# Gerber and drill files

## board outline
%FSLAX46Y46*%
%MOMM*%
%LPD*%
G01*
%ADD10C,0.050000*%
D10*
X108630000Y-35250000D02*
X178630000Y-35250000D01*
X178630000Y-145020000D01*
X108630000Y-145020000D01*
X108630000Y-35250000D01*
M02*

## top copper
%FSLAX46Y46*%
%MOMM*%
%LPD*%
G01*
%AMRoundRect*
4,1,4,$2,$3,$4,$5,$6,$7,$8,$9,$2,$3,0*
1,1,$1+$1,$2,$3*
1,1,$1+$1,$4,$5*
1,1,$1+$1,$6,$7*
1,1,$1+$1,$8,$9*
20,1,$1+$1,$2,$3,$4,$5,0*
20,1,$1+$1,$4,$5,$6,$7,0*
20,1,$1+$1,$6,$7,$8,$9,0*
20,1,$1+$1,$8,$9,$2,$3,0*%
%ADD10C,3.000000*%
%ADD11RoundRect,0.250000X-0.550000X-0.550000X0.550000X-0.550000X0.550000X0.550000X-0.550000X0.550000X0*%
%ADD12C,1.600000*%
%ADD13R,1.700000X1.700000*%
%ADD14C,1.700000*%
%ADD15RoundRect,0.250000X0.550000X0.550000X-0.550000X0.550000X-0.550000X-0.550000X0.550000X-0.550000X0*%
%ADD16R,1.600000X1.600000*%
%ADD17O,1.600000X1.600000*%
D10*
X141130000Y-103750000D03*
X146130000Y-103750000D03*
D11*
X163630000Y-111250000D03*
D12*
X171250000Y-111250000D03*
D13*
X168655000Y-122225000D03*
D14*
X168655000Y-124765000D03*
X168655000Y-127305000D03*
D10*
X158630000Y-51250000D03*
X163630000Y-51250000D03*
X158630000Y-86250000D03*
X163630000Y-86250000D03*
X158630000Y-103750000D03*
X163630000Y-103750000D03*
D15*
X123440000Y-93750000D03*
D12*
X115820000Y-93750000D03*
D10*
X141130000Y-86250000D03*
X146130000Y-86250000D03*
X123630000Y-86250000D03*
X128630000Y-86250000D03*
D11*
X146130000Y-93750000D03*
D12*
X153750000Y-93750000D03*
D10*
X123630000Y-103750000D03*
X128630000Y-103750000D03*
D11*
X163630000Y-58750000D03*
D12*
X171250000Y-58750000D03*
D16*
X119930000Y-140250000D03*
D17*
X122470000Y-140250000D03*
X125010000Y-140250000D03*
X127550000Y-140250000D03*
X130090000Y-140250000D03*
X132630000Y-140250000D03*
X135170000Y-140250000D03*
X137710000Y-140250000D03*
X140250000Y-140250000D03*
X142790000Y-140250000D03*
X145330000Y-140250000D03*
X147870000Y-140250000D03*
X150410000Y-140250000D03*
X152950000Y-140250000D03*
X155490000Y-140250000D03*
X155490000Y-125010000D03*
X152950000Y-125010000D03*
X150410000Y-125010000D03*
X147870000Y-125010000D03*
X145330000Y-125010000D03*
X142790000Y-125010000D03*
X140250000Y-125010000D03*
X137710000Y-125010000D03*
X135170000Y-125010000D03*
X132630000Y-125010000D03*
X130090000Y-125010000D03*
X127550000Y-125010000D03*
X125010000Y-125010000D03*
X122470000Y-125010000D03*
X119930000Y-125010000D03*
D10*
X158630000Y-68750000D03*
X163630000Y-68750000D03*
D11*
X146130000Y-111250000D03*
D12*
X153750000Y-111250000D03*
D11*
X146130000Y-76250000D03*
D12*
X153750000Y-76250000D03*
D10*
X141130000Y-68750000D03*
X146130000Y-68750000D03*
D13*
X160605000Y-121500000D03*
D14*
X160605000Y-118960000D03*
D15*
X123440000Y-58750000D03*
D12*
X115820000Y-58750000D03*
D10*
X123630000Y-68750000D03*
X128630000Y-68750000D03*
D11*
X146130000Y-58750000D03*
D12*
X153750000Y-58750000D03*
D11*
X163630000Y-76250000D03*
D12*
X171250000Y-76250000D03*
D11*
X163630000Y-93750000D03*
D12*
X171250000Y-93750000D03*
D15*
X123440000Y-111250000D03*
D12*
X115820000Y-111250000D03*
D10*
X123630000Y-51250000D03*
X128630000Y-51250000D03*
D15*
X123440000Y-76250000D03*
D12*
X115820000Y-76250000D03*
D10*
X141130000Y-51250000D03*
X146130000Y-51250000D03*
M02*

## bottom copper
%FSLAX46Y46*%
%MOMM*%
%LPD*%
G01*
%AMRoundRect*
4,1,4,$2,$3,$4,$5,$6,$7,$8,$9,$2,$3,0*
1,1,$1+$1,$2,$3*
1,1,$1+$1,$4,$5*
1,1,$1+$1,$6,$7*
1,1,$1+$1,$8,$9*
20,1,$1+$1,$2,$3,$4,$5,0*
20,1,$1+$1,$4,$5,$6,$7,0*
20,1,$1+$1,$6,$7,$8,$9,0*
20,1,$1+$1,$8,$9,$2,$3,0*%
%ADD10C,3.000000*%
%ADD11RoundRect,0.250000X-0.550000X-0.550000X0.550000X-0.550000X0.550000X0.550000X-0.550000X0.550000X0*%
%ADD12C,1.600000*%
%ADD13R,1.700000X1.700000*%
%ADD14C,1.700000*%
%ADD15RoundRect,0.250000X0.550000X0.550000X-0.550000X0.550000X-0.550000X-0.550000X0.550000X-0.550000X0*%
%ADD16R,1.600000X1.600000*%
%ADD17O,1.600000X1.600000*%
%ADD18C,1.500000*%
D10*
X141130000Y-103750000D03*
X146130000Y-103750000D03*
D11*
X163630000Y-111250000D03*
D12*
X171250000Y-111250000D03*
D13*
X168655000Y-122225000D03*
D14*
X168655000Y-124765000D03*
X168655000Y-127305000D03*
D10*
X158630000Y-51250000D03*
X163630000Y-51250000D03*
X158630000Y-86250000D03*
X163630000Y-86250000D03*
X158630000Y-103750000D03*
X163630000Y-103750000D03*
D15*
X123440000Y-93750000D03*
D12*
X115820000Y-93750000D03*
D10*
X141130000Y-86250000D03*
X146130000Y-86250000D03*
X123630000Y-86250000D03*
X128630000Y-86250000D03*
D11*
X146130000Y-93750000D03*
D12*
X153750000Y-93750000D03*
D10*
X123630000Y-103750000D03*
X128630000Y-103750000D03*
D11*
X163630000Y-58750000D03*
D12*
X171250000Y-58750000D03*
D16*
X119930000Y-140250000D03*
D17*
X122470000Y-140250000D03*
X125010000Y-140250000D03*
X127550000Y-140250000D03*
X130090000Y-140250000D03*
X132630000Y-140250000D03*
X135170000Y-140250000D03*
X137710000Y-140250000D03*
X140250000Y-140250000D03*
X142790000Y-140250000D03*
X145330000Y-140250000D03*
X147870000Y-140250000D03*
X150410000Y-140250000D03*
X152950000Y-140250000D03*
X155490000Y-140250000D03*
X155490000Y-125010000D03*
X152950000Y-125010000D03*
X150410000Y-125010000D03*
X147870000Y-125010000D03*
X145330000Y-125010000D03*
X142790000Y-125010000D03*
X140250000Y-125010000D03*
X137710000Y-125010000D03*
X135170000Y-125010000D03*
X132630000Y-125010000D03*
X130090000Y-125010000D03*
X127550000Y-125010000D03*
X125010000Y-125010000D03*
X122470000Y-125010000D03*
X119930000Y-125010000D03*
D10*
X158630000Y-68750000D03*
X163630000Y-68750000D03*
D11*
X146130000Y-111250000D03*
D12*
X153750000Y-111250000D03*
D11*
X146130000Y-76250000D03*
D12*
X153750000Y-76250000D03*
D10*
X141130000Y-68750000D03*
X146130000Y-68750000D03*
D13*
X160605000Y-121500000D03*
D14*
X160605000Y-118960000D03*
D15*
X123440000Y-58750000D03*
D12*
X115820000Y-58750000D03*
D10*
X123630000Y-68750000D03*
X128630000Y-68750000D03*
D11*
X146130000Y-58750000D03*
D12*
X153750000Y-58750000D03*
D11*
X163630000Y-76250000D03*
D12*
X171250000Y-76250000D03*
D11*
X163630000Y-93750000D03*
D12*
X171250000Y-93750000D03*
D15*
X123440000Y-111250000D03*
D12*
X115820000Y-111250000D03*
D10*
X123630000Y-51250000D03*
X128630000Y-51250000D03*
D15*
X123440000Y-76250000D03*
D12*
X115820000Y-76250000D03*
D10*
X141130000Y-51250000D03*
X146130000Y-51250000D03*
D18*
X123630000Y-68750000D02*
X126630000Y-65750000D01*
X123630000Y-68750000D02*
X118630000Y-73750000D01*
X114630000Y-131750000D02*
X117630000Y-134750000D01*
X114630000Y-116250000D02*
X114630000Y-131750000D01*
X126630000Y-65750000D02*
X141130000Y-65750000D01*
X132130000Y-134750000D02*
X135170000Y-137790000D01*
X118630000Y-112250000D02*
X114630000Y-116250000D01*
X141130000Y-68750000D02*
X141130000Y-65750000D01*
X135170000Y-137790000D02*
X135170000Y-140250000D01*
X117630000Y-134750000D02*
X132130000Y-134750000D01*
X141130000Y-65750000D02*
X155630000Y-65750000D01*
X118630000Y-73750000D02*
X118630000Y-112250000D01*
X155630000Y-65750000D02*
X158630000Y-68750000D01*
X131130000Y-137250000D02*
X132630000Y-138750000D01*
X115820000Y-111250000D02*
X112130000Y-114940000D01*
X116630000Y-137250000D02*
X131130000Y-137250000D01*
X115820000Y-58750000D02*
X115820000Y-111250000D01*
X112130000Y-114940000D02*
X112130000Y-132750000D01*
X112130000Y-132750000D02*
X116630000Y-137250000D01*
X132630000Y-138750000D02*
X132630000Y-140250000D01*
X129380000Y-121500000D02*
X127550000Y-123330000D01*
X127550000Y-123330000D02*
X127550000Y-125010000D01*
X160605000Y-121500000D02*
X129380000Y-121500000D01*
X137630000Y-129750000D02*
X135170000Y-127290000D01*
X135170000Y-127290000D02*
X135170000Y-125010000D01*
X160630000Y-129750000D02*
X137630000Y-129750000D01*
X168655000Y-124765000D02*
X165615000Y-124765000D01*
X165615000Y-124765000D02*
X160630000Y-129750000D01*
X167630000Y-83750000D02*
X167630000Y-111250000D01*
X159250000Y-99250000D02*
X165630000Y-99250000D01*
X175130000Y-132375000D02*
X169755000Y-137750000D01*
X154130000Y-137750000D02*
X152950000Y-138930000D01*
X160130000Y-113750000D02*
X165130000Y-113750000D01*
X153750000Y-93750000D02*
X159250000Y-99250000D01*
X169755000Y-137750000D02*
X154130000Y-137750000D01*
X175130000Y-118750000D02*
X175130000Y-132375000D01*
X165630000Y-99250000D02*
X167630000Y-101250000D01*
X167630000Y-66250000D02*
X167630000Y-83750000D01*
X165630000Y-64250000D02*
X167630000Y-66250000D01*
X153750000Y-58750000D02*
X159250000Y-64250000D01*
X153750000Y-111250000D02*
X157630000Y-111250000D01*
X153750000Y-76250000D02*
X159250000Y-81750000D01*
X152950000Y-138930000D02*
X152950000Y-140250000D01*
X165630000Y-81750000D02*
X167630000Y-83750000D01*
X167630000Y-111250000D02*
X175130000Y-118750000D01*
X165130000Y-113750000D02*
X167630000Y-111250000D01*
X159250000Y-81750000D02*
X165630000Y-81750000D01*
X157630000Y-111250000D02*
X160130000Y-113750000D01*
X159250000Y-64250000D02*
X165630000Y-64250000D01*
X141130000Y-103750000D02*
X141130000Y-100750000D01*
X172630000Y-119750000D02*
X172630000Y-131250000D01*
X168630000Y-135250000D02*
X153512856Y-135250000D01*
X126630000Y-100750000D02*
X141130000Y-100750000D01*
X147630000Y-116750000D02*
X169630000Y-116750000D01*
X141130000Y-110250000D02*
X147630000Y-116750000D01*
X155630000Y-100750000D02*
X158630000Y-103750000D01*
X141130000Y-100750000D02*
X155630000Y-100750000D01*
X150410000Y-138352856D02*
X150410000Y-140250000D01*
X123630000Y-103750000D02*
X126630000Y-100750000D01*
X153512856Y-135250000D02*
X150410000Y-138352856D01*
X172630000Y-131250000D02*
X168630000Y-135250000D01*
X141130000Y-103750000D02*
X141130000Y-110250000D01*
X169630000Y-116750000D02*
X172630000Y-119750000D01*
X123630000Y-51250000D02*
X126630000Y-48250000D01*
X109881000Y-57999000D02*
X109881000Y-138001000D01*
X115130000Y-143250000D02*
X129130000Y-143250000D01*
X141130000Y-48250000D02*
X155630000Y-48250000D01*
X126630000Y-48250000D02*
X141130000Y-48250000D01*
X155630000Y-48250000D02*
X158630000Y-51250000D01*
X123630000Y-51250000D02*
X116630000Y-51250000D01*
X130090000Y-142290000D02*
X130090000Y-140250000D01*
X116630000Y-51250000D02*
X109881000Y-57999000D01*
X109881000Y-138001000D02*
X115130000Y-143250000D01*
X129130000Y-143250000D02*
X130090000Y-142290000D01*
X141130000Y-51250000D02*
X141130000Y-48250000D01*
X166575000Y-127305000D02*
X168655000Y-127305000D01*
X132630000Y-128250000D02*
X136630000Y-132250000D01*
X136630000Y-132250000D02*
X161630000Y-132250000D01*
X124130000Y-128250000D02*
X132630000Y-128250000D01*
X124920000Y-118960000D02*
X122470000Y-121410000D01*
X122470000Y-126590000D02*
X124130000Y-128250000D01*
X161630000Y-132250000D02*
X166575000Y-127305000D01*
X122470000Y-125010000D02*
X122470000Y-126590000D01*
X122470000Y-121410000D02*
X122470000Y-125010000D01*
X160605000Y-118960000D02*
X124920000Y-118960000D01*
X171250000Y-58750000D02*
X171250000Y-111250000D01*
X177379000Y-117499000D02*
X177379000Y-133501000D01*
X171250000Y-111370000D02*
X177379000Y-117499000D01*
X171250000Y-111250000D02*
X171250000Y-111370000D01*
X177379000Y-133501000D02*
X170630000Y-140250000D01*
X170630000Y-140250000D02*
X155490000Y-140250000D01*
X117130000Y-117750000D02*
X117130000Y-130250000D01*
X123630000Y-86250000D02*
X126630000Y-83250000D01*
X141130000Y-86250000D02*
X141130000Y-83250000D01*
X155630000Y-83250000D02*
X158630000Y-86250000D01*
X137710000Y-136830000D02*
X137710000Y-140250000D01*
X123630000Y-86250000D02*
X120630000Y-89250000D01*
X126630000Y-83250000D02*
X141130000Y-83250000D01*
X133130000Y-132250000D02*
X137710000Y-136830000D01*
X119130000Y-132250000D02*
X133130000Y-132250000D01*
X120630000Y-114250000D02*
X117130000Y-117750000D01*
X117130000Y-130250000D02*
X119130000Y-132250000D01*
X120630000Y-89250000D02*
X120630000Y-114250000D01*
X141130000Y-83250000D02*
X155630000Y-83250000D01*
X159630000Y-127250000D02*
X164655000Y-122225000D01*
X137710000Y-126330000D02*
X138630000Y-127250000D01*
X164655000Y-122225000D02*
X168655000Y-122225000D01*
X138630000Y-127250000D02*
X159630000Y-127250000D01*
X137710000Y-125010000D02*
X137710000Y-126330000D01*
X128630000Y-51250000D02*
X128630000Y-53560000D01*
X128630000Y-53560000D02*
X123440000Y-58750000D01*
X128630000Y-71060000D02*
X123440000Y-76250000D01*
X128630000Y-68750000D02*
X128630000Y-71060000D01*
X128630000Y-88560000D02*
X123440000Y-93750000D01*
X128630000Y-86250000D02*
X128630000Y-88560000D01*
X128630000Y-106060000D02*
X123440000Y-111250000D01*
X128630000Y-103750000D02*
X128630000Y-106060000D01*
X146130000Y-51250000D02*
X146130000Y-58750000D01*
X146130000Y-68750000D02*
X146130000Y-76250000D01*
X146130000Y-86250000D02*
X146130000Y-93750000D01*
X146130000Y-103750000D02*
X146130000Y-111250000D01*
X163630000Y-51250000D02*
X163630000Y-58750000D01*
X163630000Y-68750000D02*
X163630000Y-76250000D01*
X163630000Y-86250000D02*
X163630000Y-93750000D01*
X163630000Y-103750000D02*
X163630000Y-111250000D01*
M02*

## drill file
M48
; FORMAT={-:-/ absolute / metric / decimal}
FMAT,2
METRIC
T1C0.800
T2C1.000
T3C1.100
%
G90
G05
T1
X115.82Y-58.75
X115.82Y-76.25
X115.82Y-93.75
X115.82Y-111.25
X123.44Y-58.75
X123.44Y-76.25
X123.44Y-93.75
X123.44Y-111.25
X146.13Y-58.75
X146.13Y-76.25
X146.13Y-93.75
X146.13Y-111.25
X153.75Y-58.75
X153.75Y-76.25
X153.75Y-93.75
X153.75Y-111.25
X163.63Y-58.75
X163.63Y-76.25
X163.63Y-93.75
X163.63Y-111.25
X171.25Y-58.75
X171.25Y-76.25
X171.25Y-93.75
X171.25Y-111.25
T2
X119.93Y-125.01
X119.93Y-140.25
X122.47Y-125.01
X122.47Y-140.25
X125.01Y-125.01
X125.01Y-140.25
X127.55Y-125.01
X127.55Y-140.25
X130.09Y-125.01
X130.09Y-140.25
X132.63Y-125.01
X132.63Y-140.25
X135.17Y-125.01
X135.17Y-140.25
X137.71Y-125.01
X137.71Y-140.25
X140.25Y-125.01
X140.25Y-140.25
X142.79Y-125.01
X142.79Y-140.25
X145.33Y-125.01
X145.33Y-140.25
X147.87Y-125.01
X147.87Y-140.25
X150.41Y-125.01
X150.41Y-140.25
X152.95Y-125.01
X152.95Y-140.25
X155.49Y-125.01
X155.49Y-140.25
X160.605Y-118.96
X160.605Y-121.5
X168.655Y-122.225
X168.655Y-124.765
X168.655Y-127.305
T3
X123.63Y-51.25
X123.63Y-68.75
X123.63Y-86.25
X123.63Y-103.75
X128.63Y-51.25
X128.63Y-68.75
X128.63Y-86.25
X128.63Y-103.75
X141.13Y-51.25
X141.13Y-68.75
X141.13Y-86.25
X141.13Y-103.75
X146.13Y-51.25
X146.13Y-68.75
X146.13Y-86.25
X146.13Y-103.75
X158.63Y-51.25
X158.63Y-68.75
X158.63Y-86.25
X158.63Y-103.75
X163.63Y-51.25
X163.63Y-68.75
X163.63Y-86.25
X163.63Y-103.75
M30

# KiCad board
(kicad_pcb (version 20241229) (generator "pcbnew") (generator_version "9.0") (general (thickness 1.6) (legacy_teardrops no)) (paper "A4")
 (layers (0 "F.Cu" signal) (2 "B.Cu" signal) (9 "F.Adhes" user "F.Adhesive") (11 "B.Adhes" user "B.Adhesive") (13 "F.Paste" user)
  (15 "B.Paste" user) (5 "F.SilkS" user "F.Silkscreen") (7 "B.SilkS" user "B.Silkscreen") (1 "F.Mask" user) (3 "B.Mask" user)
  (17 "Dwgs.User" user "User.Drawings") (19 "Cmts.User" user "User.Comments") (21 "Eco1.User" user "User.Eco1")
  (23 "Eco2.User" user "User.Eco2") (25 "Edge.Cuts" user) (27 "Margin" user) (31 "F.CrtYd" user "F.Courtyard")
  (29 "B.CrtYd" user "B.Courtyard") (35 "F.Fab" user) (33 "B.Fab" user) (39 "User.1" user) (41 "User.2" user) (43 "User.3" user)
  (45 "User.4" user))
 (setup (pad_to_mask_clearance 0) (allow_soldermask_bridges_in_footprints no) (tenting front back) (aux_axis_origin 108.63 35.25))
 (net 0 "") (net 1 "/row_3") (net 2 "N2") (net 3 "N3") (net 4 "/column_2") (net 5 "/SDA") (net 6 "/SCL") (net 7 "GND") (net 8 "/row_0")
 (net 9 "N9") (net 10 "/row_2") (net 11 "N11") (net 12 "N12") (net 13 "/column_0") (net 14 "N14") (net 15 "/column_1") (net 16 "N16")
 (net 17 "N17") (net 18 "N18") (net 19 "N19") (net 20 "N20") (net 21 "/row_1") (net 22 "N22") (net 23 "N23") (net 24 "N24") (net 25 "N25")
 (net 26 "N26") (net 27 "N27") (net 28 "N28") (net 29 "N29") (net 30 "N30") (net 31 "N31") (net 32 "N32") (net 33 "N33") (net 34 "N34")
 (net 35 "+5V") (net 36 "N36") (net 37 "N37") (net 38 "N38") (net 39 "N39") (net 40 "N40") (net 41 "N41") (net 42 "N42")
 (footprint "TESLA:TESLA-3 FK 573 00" (layer "F.Cu") (at 143.63 103.75)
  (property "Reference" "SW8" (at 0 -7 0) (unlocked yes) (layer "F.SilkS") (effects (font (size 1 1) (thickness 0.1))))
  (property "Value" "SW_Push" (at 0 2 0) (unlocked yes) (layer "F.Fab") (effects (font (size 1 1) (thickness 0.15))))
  (pad "1" thru_hole circle (at -2.5 0) (size 3 3) (drill 1.1) (layers "*.Cu" "*.Mask") (remove_unused_layers no) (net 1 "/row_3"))
  (pad "2" thru_hole circle (at 2.5 0) (size 3 3) (drill 1.1) (layers "*.Cu" "*.Mask") (remove_unused_layers no) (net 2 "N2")))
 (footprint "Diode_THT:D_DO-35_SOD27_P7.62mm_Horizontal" (layer "F.Cu") (at 163.63 111.25)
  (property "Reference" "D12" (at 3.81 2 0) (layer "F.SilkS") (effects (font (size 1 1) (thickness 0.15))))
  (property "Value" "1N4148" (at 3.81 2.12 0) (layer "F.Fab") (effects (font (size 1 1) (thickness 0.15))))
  (pad "1" thru_hole roundrect (at 0 0) (size 1.6 1.6) (drill 0.8) (layers "*.Cu" "*.Mask") (remove_unused_layers no)
   (roundrect_rratio 0.15625) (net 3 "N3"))
  (pad "2" thru_hole circle (at 7.62 0) (size 1.6 1.6) (drill 0.8) (layers "*.Cu" "*.Mask") (remove_unused_layers no) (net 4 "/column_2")))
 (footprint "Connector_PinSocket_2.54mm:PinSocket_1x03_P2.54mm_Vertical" (layer "F.Cu") (at 168.655 122.225)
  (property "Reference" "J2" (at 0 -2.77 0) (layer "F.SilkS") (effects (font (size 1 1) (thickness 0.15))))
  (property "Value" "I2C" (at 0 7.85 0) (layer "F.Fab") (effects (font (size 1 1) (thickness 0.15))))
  (pad "1" thru_hole rect (at 0 0) (size 1.7 1.7) (drill 1) (layers "*.Cu" "*.Mask") (remove_unused_layers no) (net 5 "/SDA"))
  (pad "2" thru_hole circle (at 0 2.54) (size 1.7 1.7) (drill 1) (layers "*.Cu" "*.Mask") (remove_unused_layers no) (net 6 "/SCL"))
  (pad "3" thru_hole circle (at 0 5.08) (size 1.7 1.7) (drill 1) (layers "*.Cu" "*.Mask") (remove_unused_layers no) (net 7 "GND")))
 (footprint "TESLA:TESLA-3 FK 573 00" (layer "F.Cu") (at 161.13 51.25)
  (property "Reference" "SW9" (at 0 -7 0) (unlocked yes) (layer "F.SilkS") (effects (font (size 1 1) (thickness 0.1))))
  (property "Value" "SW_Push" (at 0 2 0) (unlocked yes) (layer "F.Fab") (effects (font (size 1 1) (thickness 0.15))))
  (pad "1" thru_hole circle (at -2.5 0) (size 3 3) (drill 1.1) (layers "*.Cu" "*.Mask") (remove_unused_layers no) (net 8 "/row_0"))
  (pad "2" thru_hole circle (at 2.5 0) (size 3 3) (drill 1.1) (layers "*.Cu" "*.Mask") (remove_unused_layers no) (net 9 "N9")))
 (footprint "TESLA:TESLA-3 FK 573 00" (layer "F.Cu") (at 161.13 86.25)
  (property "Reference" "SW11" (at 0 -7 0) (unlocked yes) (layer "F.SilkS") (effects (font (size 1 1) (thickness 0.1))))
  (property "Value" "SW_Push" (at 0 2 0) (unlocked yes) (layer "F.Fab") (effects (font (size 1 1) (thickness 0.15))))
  (pad "1" thru_hole circle (at -2.5 0) (size 3 3) (drill 1.1) (layers "*.Cu" "*.Mask") (remove_unused_layers no) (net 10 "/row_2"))
  (pad "2" thru_hole circle (at 2.5 0) (size 3 3) (drill 1.1) (layers "*.Cu" "*.Mask") (remove_unused_layers no) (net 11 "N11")))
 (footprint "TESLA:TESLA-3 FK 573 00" (layer "F.Cu") (at 161.13 103.75)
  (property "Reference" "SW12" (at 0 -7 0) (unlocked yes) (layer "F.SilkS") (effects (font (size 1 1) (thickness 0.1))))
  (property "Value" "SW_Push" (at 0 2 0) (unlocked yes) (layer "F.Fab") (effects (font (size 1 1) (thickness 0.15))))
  (pad "1" thru_hole circle (at -2.5 0) (size 3 3) (drill 1.1) (layers "*.Cu" "*.Mask") (remove_unused_layers no) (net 1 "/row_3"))
  (pad "2" thru_hole circle (at 2.5 0) (size 3 3) (drill 1.1) (layers "*.Cu" "*.Mask") (remove_unused_layers no) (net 3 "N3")))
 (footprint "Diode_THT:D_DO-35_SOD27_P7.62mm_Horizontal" (layer "F.Cu") (at 123.44 93.75 180)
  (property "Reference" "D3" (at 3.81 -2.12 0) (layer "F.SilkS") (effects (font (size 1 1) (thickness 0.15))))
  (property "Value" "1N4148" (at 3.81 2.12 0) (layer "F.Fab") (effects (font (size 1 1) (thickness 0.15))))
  (pad "1" thru_hole roundrect (at 0 0 180) (size 1.6 1.6) (drill 0.8) (layers "*.Cu" "*.Mask") (remove_unused_layers no)
   (roundrect_rratio 0.15625) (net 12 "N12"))
  (pad "2" thru_hole circle (at 7.62 0 180) (size 1.6 1.6) (drill 0.8) (layers "*.Cu" "*.Mask") (remove_unused_layers no)
   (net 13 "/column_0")))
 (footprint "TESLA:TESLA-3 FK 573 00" (layer "F.Cu") (at 143.63 86.25)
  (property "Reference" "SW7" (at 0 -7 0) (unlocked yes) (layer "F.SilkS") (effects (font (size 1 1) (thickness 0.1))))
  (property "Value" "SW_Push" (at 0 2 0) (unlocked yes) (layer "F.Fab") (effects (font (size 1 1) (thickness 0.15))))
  (pad "1" thru_hole circle (at -2.5 0) (size 3 3) (drill 1.1) (layers "*.Cu" "*.Mask") (remove_unused_layers no) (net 10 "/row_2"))
  (pad "2" thru_hole circle (at 2.5 0) (size 3 3) (drill 1.1) (layers "*.Cu" "*.Mask") (remove_unused_layers no) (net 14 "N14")))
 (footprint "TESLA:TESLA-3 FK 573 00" (layer "F.Cu") (at 126.13 86.25)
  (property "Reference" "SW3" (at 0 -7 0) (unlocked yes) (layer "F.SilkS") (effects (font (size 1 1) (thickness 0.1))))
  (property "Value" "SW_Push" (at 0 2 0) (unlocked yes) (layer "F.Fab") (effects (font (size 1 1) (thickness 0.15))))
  (pad "1" thru_hole circle (at -2.5 0) (size 3 3) (drill 1.1) (layers "*.Cu" "*.Mask") (remove_unused_layers no) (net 10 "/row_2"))
  (pad "2" thru_hole circle (at 2.5 0) (size 3 3) (drill 1.1) (layers "*.Cu" "*.Mask") (remove_unused_layers no) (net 12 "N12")))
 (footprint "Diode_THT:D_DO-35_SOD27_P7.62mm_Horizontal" (layer "F.Cu") (at 146.13 93.75)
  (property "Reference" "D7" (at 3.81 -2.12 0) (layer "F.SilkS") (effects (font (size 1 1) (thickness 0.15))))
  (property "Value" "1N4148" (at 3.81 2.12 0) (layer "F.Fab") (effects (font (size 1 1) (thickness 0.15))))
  (pad "1" thru_hole roundrect (at 0 0) (size 1.6 1.6) (drill 0.8) (layers "*.Cu" "*.Mask") (remove_unused_layers no)
   (roundrect_rratio 0.15625) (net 14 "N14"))
  (pad "2" thru_hole circle (at 7.62 0) (size 1.6 1.6) (drill 0.8) (layers "*.Cu" "*.Mask") (remove_unused_layers no) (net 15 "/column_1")))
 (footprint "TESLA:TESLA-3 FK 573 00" (layer "F.Cu") (at 126.13 103.75)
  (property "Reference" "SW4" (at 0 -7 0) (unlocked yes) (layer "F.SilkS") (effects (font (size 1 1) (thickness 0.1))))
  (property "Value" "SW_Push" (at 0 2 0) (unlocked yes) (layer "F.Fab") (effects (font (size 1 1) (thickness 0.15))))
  (pad "1" thru_hole circle (at -2.5 0) (size 3 3) (drill 1.1) (layers "*.Cu" "*.Mask") (remove_unused_layers no) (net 1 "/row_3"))
  (pad "2" thru_hole circle (at 2.5 0) (size 3 3) (drill 1.1) (layers "*.Cu" "*.Mask") (remove_unused_layers no) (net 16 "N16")))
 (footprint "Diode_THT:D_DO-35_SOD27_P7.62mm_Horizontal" (layer "F.Cu") (at 163.63 58.75)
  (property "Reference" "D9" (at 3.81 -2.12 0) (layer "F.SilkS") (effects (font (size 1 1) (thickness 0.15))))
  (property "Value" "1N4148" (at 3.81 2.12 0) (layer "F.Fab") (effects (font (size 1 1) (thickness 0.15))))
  (pad "1" thru_hole roundrect (at 0 0) (size 1.6 1.6) (drill 0.8) (layers "*.Cu" "*.Mask") (remove_unused_layers no)
   (roundrect_rratio 0.15625) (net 9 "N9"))
  (pad "2" thru_hole circle (at 7.62 0) (size 1.6 1.6) (drill 0.8) (layers "*.Cu" "*.Mask") (remove_unused_layers no) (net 4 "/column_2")))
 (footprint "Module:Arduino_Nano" (layer "F.Cu") (at 119.93 140.25 90)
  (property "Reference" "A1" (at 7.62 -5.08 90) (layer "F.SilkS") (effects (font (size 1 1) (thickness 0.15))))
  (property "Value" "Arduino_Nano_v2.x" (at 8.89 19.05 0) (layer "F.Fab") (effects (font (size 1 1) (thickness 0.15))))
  (pad "1" thru_hole rect (at 0 0 90) (size 1.6 1.6) (drill 1) (layers "*.Cu" "*.Mask") (remove_unused_layers no) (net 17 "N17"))
  (pad "2" thru_hole oval (at 0 2.54 90) (size 1.6 1.6) (drill 1) (layers "*.Cu" "*.Mask") (remove_unused_layers no) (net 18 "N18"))
  (pad "3" thru_hole oval (at 0 5.08 90) (size 1.6 1.6) (drill 1) (layers "*.Cu" "*.Mask") (remove_unused_layers no) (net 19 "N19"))
  (pad "4" thru_hole oval (at 0 7.62 90) (size 1.6 1.6) (drill 1) (layers "*.Cu" "*.Mask") (remove_unused_layers no) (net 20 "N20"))
  (pad "5" thru_hole oval (at 0 10.16 90) (size 1.6 1.6) (drill 1) (layers "*.Cu" "*.Mask") (remove_unused_layers no) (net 8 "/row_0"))
  (pad "6" thru_hole oval (at 0 12.7 90) (size 1.6 1.6) (drill 1) (layers "*.Cu" "*.Mask") (remove_unused_layers no) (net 13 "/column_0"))
  (pad "7" thru_hole oval (at 0 15.24 90) (size 1.6 1.6) (drill 1) (layers "*.Cu" "*.Mask") (remove_unused_layers no) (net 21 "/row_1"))
  (pad "8" thru_hole oval (at 0 17.78 90) (size 1.6 1.6) (drill 1) (layers "*.Cu" "*.Mask") (remove_unused_layers no) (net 10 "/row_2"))
  (pad "9" thru_hole oval (at 0 20.32 90) (size 1.6 1.6) (drill 1) (layers "*.Cu" "*.Mask") (remove_unused_layers no) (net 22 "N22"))
  (pad "10" thru_hole oval (at 0 22.86 90) (size 1.6 1.6) (drill 1) (layers "*.Cu" "*.Mask") (remove_unused_layers no) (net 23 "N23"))
  (pad "11" thru_hole oval (at 0 25.4 90) (size 1.6 1.6) (drill 1) (layers "*.Cu" "*.Mask") (remove_unused_layers no) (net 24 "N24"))
  (pad "12" thru_hole oval (at 0 27.94 90) (size 1.6 1.6) (drill 1) (layers "*.Cu" "*.Mask") (remove_unused_layers no) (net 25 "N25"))
  (pad "13" thru_hole oval (at 0 30.48 90) (size 1.6 1.6) (drill 1) (layers "*.Cu" "*.Mask") (remove_unused_layers no) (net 1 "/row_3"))
  (pad "14" thru_hole oval (at 0 33.02 90) (size 1.6 1.6) (drill 1) (layers "*.Cu" "*.Mask") (remove_unused_layers no) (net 15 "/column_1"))
  (pad "15" thru_hole oval (at 0 35.56 90) (size 1.6 1.6) (drill 1) (layers "*.Cu" "*.Mask") (remove_unused_layers no) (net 4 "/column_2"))
  (pad "16" thru_hole oval (at 15.24 35.56 90) (size 1.6 1.6) (drill 1) (layers "*.Cu" "*.Mask") (remove_unused_layers no) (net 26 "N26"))
  (pad "17" thru_hole oval (at 15.24 33.02 90) (size 1.6 1.6) (drill 1) (layers "*.Cu" "*.Mask") (remove_unused_layers no) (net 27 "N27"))
  (pad "18" thru_hole oval (at 15.24 30.48 90) (size 1.6 1.6) (drill 1) (layers "*.Cu" "*.Mask") (remove_unused_layers no) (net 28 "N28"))
  (pad "19" thru_hole oval (at 15.24 27.94 90) (size 1.6 1.6) (drill 1) (layers "*.Cu" "*.Mask") (remove_unused_layers no) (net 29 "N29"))
  (pad "20" thru_hole oval (at 15.24 25.4 90) (size 1.6 1.6) (drill 1) (layers "*.Cu" "*.Mask") (remove_unused_layers no) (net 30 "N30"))
  (pad "21" thru_hole oval (at 15.24 22.86 90) (size 1.6 1.6) (drill 1) (layers "*.Cu" "*.Mask") (remove_unused_layers no) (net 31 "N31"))
  (pad "22" thru_hole oval (at 15.24 20.32 90) (size 1.6 1.6) (drill 1) (layers "*.Cu" "*.Mask") (remove_unused_layers no) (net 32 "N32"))
  (pad "23" thru_hole oval (at 15.24 17.78 90) (size 1.6 1.6) (drill 1) (layers "*.Cu" "*.Mask") (remove_unused_layers no) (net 5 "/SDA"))
  (pad "24" thru_hole oval (at 15.24 15.24 90) (size 1.6 1.6) (drill 1) (layers "*.Cu" "*.Mask") (remove_unused_layers no) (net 6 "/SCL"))
  (pad "25" thru_hole oval (at 15.24 12.7 90) (size 1.6 1.6) (drill 1) (layers "*.Cu" "*.Mask") (remove_unused_layers no) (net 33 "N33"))
  (pad "26" thru_hole oval (at 15.24 10.16 90) (size 1.6 1.6) (drill 1) (layers "*.Cu" "*.Mask") (remove_unused_layers no) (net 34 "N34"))
  (pad "27" thru_hole oval (at 15.24 7.62 90) (size 1.6 1.6) (drill 1) (layers "*.Cu" "*.Mask") (remove_unused_layers no) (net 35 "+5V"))
  (pad "28" thru_hole oval (at 15.24 5.08 90) (size 1.6 1.6) (drill 1) (layers "*.Cu" "*.Mask") (remove_unused_layers no) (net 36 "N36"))
  (pad "29" thru_hole oval (at 15.24 2.54 90) (size 1.6 1.6) (drill 1) (layers "*.Cu" "*.Mask") (remove_unused_layers no) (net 7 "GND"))
  (pad "30" thru_hole oval (at 15.24 0 90) (size 1.6 1.6) (drill 1) (layers "*.Cu" "*.Mask") (remove_unused_layers no) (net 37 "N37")))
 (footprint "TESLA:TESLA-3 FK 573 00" (layer "F.Cu") (at 161.13 68.75)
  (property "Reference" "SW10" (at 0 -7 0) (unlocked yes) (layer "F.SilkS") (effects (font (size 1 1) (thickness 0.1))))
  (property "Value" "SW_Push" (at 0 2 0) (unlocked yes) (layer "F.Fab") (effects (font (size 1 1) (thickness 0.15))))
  (pad "1" thru_hole circle (at -2.5 0) (size 3 3) (drill 1.1) (layers "*.Cu" "*.Mask") (remove_unused_layers no) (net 21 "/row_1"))
  (pad "2" thru_hole circle (at 2.5 0) (size 3 3) (drill 1.1) (layers "*.Cu" "*.Mask") (remove_unused_layers no) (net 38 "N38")))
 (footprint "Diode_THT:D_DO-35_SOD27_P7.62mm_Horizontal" (layer "F.Cu") (at 146.13 111.25)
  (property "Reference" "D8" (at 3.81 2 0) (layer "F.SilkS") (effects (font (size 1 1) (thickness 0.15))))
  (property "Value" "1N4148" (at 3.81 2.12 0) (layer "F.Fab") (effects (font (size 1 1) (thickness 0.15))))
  (pad "1" thru_hole roundrect (at 0 0) (size 1.6 1.6) (drill 0.8) (layers "*.Cu" "*.Mask") (remove_unused_layers no)
   (roundrect_rratio 0.15625) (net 2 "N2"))
  (pad "2" thru_hole circle (at 7.62 0) (size 1.6 1.6) (drill 0.8) (layers "*.Cu" "*.Mask") (remove_unused_layers no) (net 15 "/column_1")))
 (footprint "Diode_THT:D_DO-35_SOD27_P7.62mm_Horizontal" (layer "F.Cu") (at 146.13 76.25)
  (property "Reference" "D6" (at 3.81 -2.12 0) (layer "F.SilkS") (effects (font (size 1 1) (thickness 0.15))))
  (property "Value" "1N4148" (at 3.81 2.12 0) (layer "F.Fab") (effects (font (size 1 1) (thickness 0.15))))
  (pad "1" thru_hole roundrect (at 0 0) (size 1.6 1.6) (drill 0.8) (layers "*.Cu" "*.Mask") (remove_unused_layers no)
   (roundrect_rratio 0.15625) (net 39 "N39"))
  (pad "2" thru_hole circle (at 7.62 0) (size 1.6 1.6) (drill 0.8) (layers "*.Cu" "*.Mask") (remove_unused_layers no) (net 15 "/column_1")))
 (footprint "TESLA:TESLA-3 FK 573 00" (layer "F.Cu") (at 143.63 68.75)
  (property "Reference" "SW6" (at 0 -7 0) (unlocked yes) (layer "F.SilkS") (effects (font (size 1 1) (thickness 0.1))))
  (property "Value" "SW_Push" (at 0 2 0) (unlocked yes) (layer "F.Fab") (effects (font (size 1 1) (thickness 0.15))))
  (pad "1" thru_hole circle (at -2.5 0) (size 3 3) (drill 1.1) (layers "*.Cu" "*.Mask") (remove_unused_layers no) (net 21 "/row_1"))
  (pad "2" thru_hole circle (at 2.5 0) (size 3 3) (drill 1.1) (layers "*.Cu" "*.Mask") (remove_unused_layers no) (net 39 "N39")))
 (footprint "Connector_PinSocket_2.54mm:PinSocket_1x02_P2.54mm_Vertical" (layer "F.Cu") (at 160.605 121.5 180)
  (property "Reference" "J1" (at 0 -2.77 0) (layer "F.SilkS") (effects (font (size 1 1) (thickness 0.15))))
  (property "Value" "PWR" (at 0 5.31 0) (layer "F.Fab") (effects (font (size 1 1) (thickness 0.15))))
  (pad "1" thru_hole rect (at 0 0 180) (size 1.7 1.7) (drill 1) (layers "*.Cu" "*.Mask") (remove_unused_layers no) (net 35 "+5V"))
  (pad "2" thru_hole circle (at 0 2.54 180) (size 1.7 1.7) (drill 1) (layers "*.Cu" "*.Mask") (remove_unused_layers no) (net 7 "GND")))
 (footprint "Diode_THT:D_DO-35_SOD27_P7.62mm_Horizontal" (layer "F.Cu") (at 123.44 58.75 180)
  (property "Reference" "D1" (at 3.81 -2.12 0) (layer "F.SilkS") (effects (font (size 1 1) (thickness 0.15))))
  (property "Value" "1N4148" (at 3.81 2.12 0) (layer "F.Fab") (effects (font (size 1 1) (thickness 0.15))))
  (pad "1" thru_hole roundrect (at 0 0 180) (size 1.6 1.6) (drill 0.8) (layers "*.Cu" "*.Mask") (remove_unused_layers no)
   (roundrect_rratio 0.15625) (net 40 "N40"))
  (pad "2" thru_hole circle (at 7.62 0 180) (size 1.6 1.6) (drill 0.8) (layers "*.Cu" "*.Mask") (remove_unused_layers no)
   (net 13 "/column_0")))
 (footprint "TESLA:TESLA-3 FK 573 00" (layer "F.Cu") (at 126.13 68.75)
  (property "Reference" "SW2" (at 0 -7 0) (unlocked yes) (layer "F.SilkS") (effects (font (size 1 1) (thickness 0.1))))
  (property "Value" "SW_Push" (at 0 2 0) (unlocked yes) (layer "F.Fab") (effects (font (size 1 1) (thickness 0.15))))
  (pad "1" thru_hole circle (at -2.5 0) (size 3 3) (drill 1.1) (layers "*.Cu" "*.Mask") (remove_unused_layers no) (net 21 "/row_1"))
  (pad "2" thru_hole circle (at 2.5 0) (size 3 3) (drill 1.1) (layers "*.Cu" "*.Mask") (remove_unused_layers no) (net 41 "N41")))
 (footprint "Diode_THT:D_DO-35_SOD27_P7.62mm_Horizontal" (layer "F.Cu") (at 146.13 58.75)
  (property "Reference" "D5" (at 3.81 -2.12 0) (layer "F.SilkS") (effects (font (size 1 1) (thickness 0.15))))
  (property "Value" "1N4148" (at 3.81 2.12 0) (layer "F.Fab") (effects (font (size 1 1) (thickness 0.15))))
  (pad "1" thru_hole roundrect (at 0 0) (size 1.6 1.6) (drill 0.8) (layers "*.Cu" "*.Mask") (remove_unused_layers no)
   (roundrect_rratio 0.15625) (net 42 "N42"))
  (pad "2" thru_hole circle (at 7.62 0) (size 1.6 1.6) (drill 0.8) (layers "*.Cu" "*.Mask") (remove_unused_layers no) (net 15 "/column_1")))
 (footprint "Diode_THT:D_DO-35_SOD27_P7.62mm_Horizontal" (layer "F.Cu") (at 163.63 76.25)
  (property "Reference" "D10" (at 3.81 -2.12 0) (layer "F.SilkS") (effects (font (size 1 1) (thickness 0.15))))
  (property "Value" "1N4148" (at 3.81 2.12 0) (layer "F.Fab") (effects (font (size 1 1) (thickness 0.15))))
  (pad "1" thru_hole roundrect (at 0 0) (size 1.6 1.6) (drill 0.8) (layers "*.Cu" "*.Mask") (remove_unused_layers no)
   (roundrect_rratio 0.15625) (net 38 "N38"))
  (pad "2" thru_hole circle (at 7.62 0) (size 1.6 1.6) (drill 0.8) (layers "*.Cu" "*.Mask") (remove_unused_layers no) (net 4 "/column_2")))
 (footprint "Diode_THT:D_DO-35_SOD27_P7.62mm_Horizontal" (layer "F.Cu") (at 163.63 93.75)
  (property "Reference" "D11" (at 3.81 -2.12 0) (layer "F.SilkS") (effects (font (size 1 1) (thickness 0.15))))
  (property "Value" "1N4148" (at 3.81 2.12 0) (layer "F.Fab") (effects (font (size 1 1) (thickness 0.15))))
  (pad "1" thru_hole roundrect (at 0 0) (size 1.6 1.6) (drill 0.8) (layers "*.Cu" "*.Mask") (remove_unused_layers no)
   (roundrect_rratio 0.15625) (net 11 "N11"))
  (pad "2" thru_hole circle (at 7.62 0) (size 1.6 1.6) (drill 0.8) (layers "*.Cu" "*.Mask") (remove_unused_layers no) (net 4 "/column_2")))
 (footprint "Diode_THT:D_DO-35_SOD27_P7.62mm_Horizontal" (layer "F.Cu") (at 123.44 111.25 180)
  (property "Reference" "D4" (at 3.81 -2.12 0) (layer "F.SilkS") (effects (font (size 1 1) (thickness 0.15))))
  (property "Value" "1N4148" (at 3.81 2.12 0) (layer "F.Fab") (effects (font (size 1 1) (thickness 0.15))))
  (pad "1" thru_hole roundrect (at 0 0 180) (size 1.6 1.6) (drill 0.8) (layers "*.Cu" "*.Mask") (remove_unused_layers no)
   (roundrect_rratio 0.15625) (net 16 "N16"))
  (pad "2" thru_hole circle (at 7.62 0 180) (size 1.6 1.6) (drill 0.8) (layers "*.Cu" "*.Mask") (remove_unused_layers no)
   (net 13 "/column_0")))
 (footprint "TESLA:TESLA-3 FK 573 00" (layer "F.Cu") (at 126.13 51.25)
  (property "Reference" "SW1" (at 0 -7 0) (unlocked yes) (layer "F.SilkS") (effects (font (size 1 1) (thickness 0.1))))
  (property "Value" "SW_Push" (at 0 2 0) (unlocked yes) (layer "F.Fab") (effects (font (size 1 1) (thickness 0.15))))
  (pad "1" thru_hole circle (at -2.5 0) (size 3 3) (drill 1.1) (layers "*.Cu" "*.Mask") (remove_unused_layers no) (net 8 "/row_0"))
  (pad "2" thru_hole circle (at 2.5 0) (size 3 3) (drill 1.1) (layers "*.Cu" "*.Mask") (remove_unused_layers no) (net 40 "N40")))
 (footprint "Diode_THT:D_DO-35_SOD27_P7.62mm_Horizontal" (layer "F.Cu") (at 123.44 76.25 180)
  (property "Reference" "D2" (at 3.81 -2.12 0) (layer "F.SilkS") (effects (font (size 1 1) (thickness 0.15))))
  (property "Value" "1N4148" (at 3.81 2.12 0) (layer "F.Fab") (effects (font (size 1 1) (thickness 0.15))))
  (pad "1" thru_hole roundrect (at 0 0 180) (size 1.6 1.6) (drill 0.8) (layers "*.Cu" "*.Mask") (remove_unused_layers no)
   (roundrect_rratio 0.15625) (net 41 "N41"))
  (pad "2" thru_hole circle (at 7.62 0 180) (size 1.6 1.6) (drill 0.8) (layers "*.Cu" "*.Mask") (remove_unused_layers no)
   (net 13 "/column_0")))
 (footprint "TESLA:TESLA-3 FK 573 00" (layer "F.Cu") (at 143.63 51.25)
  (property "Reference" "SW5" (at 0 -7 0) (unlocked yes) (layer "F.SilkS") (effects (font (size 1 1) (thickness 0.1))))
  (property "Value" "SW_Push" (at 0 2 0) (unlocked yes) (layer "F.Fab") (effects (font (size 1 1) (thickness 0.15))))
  (pad "1" thru_hole circle (at -2.5 0) (size 3 3) (drill 1.1) (layers "*.Cu" "*.Mask") (remove_unused_layers no) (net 8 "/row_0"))
  (pad "2" thru_hole circle (at 2.5 0) (size 3 3) (drill 1.1) (layers "*.Cu" "*.Mask") (remove_unused_layers no) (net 42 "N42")))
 (gr_rect (start 108.63 35.25) (end 178.63 145.02) (stroke (width 0.05) (type solid)) (fill no) (layer "Edge.Cuts"))
 (segment (start 123.63 68.75) (end 126.63 65.75) (width 1.5) (layer "B.Cu") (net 21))
 (segment (start 123.63 68.75) (end 118.63 73.75) (width 1.5) (layer "B.Cu") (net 21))
 (segment (start 114.63 131.75) (end 117.63 134.75) (width 1.5) (layer "B.Cu") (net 21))
 (segment (start 114.63 116.25) (end 114.63 131.75) (width 1.5) (layer "B.Cu") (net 21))
 (segment (start 126.63 65.75) (end 141.13 65.75) (width 1.5) (layer "B.Cu") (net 21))
 (segment (start 132.13 134.75) (end 135.17 137.79) (width 1.5) (layer "B.Cu") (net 21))
 (segment (start 118.63 112.25) (end 114.63 116.25) (width 1.5) (layer "B.Cu") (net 21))
 (segment (start 141.13 68.75) (end 141.13 65.75) (width 1.5) (layer "B.Cu") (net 21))
 (segment (start 135.17 137.79) (end 135.17 140.25) (width 1.5) (layer "B.Cu") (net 21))
 (segment (start 117.63 134.75) (end 132.13 134.75) (width 1.5) (layer "B.Cu") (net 21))
 (segment (start 141.13 65.75) (end 155.63 65.75) (width 1.5) (layer "B.Cu") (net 21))
 (segment (start 118.63 73.75) (end 118.63 112.25) (width 1.5) (layer "B.Cu") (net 21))
 (segment (start 155.63 65.75) (end 158.63 68.75) (width 1.5) (layer "B.Cu") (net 21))
 (segment (start 131.13 137.25) (end 132.63 138.75) (width 1.5) (layer "B.Cu") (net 13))
 (segment (start 115.82 111.25) (end 112.13 114.94) (width 1.5) (layer "B.Cu") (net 13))
 (segment (start 116.63 137.25) (end 131.13 137.25) (width 1.5) (layer "B.Cu") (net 13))
 (segment (start 115.82 58.75) (end 115.82 111.25) (width 1.5) (layer "B.Cu") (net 13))
 (segment (start 112.13 114.94) (end 112.13 132.75) (width 1.5) (layer "B.Cu") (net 13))
 (segment (start 112.13 132.75) (end 116.63 137.25) (width 1.5) (layer "B.Cu") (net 13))
 (segment (start 132.63 138.75) (end 132.63 140.25) (width 1.5) (layer "B.Cu") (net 13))
 (segment (start 129.38 121.5) (end 127.55 123.33) (width 1.5) (layer "B.Cu") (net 35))
 (segment (start 127.55 123.33) (end 127.55 125.01) (width 1.5) (layer "B.Cu") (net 35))
 (segment (start 160.605 121.5) (end 129.38 121.5) (width 1.5) (layer "B.Cu") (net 35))
 (segment (start 137.63 129.75) (end 135.17 127.29) (width 1.5) (layer "B.Cu") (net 6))
 (segment (start 135.17 127.29) (end 135.17 125.01) (width 1.5) (layer "B.Cu") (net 6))
 (segment (start 160.63 129.75) (end 137.63 129.75) (width 1.5) (layer "B.Cu") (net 6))
 (segment (start 168.655 124.765) (end 165.615 124.765) (width 1.5) (layer "B.Cu") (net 6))
 (segment (start 165.615 124.765) (end 160.63 129.75) (width 1.5) (layer "B.Cu") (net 6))
 (segment (start 167.63 83.75) (end 167.63 111.25) (width 1.5) (layer "B.Cu") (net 15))
 (segment (start 159.25 99.25) (end 165.63 99.25) (width 1.5) (layer "B.Cu") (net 15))
 (segment (start 175.13 132.375) (end 169.755 137.75) (width 1.5) (layer "B.Cu") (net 15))
 (segment (start 154.13 137.75) (end 152.95 138.93) (width 1.5) (layer "B.Cu") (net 15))
 (segment (start 160.13 113.75) (end 165.13 113.75) (width 1.5) (layer "B.Cu") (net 15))
 (segment (start 153.75 93.75) (end 159.25 99.25) (width 1.5) (layer "B.Cu") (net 15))
 (segment (start 169.755 137.75) (end 154.13 137.75) (width 1.5) (layer "B.Cu") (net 15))
 (segment (start 175.13 118.75) (end 175.13 132.375) (width 1.5) (layer "B.Cu") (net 15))
 (segment (start 165.63 99.25) (end 167.63 101.25) (width 1.5) (layer "B.Cu") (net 15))
 (segment (start 167.63 66.25) (end 167.63 83.75) (width 1.5) (layer "B.Cu") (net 15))
 (segment (start 165.63 64.25) (end 167.63 66.25) (width 1.5) (layer "B.Cu") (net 15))
 (segment (start 153.75 58.75) (end 159.25 64.25) (width 1.5) (layer "B.Cu") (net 15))
 (segment (start 153.75 111.25) (end 157.63 111.25) (width 1.5) (layer "B.Cu") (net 15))
 (segment (start 153.75 76.25) (end 159.25 81.75) (width 1.5) (layer "B.Cu") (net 15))
 (segment (start 152.95 138.93) (end 152.95 140.25) (width 1.5) (layer "B.Cu") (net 15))
 (segment (start 165.63 81.75) (end 167.63 83.75) (width 1.5) (layer "B.Cu") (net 15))
 (segment (start 167.63 111.25) (end 175.13 118.75) (width 1.5) (layer "B.Cu") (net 15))
 (segment (start 165.13 113.75) (end 167.63 111.25) (width 1.5) (layer "B.Cu") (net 15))
 (segment (start 159.25 81.75) (end 165.63 81.75) (width 1.5) (layer "B.Cu") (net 15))
 (segment (start 157.63 111.25) (end 160.13 113.75) (width 1.5) (layer "B.Cu") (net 15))
 (segment (start 159.25 64.25) (end 165.63 64.25) (width 1.5) (layer "B.Cu") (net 15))
 (segment (start 141.13 103.75) (end 141.13 100.75) (width 1.5) (layer "B.Cu") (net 1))
 (segment (start 172.63 119.75) (end 172.63 131.25) (width 1.5) (layer "B.Cu") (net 1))
 (segment (start 168.63 135.25) (end 153.512856 135.25) (width 1.5) (layer "B.Cu") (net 1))
 (segment (start 126.63 100.75) (end 141.13 100.75) (width 1.5) (layer "B.Cu") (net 1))
 (segment (start 147.63 116.75) (end 169.63 116.75) (width 1.5) (layer "B.Cu") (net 1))
 (segment (start 141.13 110.25) (end 147.63 116.75) (width 1.5) (layer "B.Cu") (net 1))
 (segment (start 155.63 100.75) (end 158.63 103.75) (width 1.5) (layer "B.Cu") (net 1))
 (segment (start 141.13 100.75) (end 155.63 100.75) (width 1.5) (layer "B.Cu") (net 1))
 (segment (start 150.41 138.352856) (end 150.41 140.25) (width 1.5) (layer "B.Cu") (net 1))
 (segment (start 123.63 103.75) (end 126.63 100.75) (width 1.5) (layer "B.Cu") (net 1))
 (segment (start 153.512856 135.25) (end 150.41 138.352856) (width 1.5) (layer "B.Cu") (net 1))
 (segment (start 172.63 131.25) (end 168.63 135.25) (width 1.5) (layer "B.Cu") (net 1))
 (segment (start 141.13 103.75) (end 141.13 110.25) (width 1.5) (layer "B.Cu") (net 1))
 (segment (start 169.63 116.75) (end 172.63 119.75) (width 1.5) (layer "B.Cu") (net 1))
 (segment (start 123.63 51.25) (end 126.63 48.25) (width 1.5) (layer "B.Cu") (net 8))
 (segment (start 109.881 57.999) (end 109.881 138.001) (width 1.5) (layer "B.Cu") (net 8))
 (segment (start 115.13 143.25) (end 129.13 143.25) (width 1.5) (layer "B.Cu") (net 8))
 (segment (start 141.13 48.25) (end 155.63 48.25) (width 1.5) (layer "B.Cu") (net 8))
 (segment (start 126.63 48.25) (end 141.13 48.25) (width 1.5) (layer "B.Cu") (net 8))
 (segment (start 155.63 48.25) (end 158.63 51.25) (width 1.5) (layer "B.Cu") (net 8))
 (segment (start 123.63 51.25) (end 116.63 51.25) (width 1.5) (layer "B.Cu") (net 8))
 (segment (start 130.09 142.29) (end 130.09 140.25) (width 1.5) (layer "B.Cu") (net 8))
 (segment (start 116.63 51.25) (end 109.881 57.999) (width 1.5) (layer "B.Cu") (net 8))
 (segment (start 109.881 138.001) (end 115.13 143.25) (width 1.5) (layer "B.Cu") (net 8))
 (segment (start 129.13 143.25) (end 130.09 142.29) (width 1.5) (layer "B.Cu") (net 8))
 (segment (start 141.13 51.25) (end 141.13 48.25) (width 1.5) (layer "B.Cu") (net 8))
 (segment (start 166.575 127.305) (end 168.655 127.305) (width 1.5) (layer "B.Cu") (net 7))
 (segment (start 132.63 128.25) (end 136.63 132.25) (width 1.5) (layer "B.Cu") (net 7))
 (segment (start 136.63 132.25) (end 161.63 132.25) (width 1.5) (layer "B.Cu") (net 7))
 (segment (start 124.13 128.25) (end 132.63 128.25) (width 1.5) (layer "B.Cu") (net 7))
 (segment (start 124.92 118.96) (end 122.47 121.41) (width 1.5) (layer "B.Cu") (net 7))
 (segment (start 122.47 126.59) (end 124.13 128.25) (width 1.5) (layer "B.Cu") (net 7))
 (segment (start 161.63 132.25) (end 166.575 127.305) (width 1.5) (layer "B.Cu") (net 7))
 (segment (start 122.47 125.01) (end 122.47 126.59) (width 1.5) (layer "B.Cu") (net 7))
 (segment (start 122.47 121.41) (end 122.47 125.01) (width 1.5) (layer "B.Cu") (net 7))
 (segment (start 160.605 118.96) (end 124.92 118.96) (width 1.5) (layer "B.Cu") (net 7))
 (segment (start 171.25 58.75) (end 171.25 111.25) (width 1.5) (layer "B.Cu") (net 4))
 (segment (start 177.379 117.499) (end 177.379 133.501) (width 1.5) (layer "B.Cu") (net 4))
 (segment (start 171.25 111.37) (end 177.379 117.499) (width 1.5) (layer "B.Cu") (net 4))
 (segment (start 171.25 111.25) (end 171.25 111.37) (width 1.5) (layer "B.Cu") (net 4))
 (segment (start 177.379 133.501) (end 170.63 140.25) (width 1.5) (layer "B.Cu") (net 4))
 (segment (start 170.63 140.25) (end 155.49 140.25) (width 1.5) (layer "B.Cu") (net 4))
 (segment (start 117.13 117.75) (end 117.13 130.25) (width 1.5) (layer "B.Cu") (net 10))
 (segment (start 123.63 86.25) (end 126.63 83.25) (width 1.5) (layer "B.Cu") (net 10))
 (segment (start 141.13 86.25) (end 141.13 83.25) (width 1.5) (layer "B.Cu") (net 10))
 (segment (start 155.63 83.25) (end 158.63 86.25) (width 1.5) (layer "B.Cu") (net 10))
 (segment (start 137.71 136.83) (end 137.71 140.25) (width 1.5) (layer "B.Cu") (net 10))
 (segment (start 123.63 86.25) (end 120.63 89.25) (width 1.5) (layer "B.Cu") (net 10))
 (segment (start 126.63 83.25) (end 141.13 83.25) (width 1.5) (layer "B.Cu") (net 10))
 (segment (start 133.13 132.25) (end 137.71 136.83) (width 1.5) (layer "B.Cu") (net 10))
 (segment (start 119.13 132.25) (end 133.13 132.25) (width 1.5) (layer "B.Cu") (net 10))
 (segment (start 120.63 114.25) (end 117.13 117.75) (width 1.5) (layer "B.Cu") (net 10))
 (segment (start 117.13 130.25) (end 119.13 132.25) (width 1.5) (layer "B.Cu") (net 10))
 (segment (start 120.63 89.25) (end 120.63 114.25) (width 1.5) (layer "B.Cu") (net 10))
 (segment (start 141.13 83.25) (end 155.63 83.25) (width 1.5) (layer "B.Cu") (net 10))
 (segment (start 159.63 127.25) (end 164.655 122.225) (width 1.5) (layer "B.Cu") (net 5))
 (segment (start 137.71 126.33) (end 138.63 127.25) (width 1.5) (layer "B.Cu") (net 5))
 (segment (start 164.655 122.225) (end 168.655 122.225) (width 1.5) (layer "B.Cu") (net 5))
 (segment (start 138.63 127.25) (end 159.63 127.25) (width 1.5) (layer "B.Cu") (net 5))
 (segment (start 137.71 125.01) (end 137.71 126.33) (width 1.5) (layer "B.Cu") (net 5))
 (segment (start 128.63 51.25) (end 128.63 53.56) (width 1.5) (layer "B.Cu") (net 40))
 (segment (start 128.63 53.56) (end 123.44 58.75) (width 1.5) (layer "B.Cu") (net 40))
 (segment (start 128.63 71.06) (end 123.44 76.25) (width 1.5) (layer "B.Cu") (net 41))
 (segment (start 128.63 68.75) (end 128.63 71.06) (width 1.5) (layer "B.Cu") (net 41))
 (segment (start 128.63 88.56) (end 123.44 93.75) (width 1.5) (layer "B.Cu") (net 12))
 (segment (start 128.63 86.25) (end 128.63 88.56) (width 1.5) (layer "B.Cu") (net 12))
 (segment (start 128.63 106.06) (end 123.44 111.25) (width 1.5) (layer "B.Cu") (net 16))
 (segment (start 128.63 103.75) (end 128.63 106.06) (width 1.5) (layer "B.Cu") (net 16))
 (segment (start 146.13 51.25) (end 146.13 58.75) (width 1.5) (layer "B.Cu") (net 42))
 (segment (start 146.13 68.75) (end 146.13 76.25) (width 1.5) (layer "B.Cu") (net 39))
 (segment (start 146.13 86.25) (end 146.13 93.75) (width 1.5) (layer "B.Cu") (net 14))
 (segment (start 146.13 103.75) (end 146.13 111.25) (width 1.5) (layer "B.Cu") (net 2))
 (segment (start 163.63 51.25) (end 163.63 58.75) (width 1.5) (layer "B.Cu") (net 9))
 (segment (start 163.63 68.75) (end 163.63 76.25) (width 1.5) (layer "B.Cu") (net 38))
 (segment (start 163.63 86.25) (end 163.63 93.75) (width 1.5) (layer "B.Cu") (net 11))
 (segment (start 163.63 103.75) (end 163.63 111.25) (width 1.5) (layer "B.Cu") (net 3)))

